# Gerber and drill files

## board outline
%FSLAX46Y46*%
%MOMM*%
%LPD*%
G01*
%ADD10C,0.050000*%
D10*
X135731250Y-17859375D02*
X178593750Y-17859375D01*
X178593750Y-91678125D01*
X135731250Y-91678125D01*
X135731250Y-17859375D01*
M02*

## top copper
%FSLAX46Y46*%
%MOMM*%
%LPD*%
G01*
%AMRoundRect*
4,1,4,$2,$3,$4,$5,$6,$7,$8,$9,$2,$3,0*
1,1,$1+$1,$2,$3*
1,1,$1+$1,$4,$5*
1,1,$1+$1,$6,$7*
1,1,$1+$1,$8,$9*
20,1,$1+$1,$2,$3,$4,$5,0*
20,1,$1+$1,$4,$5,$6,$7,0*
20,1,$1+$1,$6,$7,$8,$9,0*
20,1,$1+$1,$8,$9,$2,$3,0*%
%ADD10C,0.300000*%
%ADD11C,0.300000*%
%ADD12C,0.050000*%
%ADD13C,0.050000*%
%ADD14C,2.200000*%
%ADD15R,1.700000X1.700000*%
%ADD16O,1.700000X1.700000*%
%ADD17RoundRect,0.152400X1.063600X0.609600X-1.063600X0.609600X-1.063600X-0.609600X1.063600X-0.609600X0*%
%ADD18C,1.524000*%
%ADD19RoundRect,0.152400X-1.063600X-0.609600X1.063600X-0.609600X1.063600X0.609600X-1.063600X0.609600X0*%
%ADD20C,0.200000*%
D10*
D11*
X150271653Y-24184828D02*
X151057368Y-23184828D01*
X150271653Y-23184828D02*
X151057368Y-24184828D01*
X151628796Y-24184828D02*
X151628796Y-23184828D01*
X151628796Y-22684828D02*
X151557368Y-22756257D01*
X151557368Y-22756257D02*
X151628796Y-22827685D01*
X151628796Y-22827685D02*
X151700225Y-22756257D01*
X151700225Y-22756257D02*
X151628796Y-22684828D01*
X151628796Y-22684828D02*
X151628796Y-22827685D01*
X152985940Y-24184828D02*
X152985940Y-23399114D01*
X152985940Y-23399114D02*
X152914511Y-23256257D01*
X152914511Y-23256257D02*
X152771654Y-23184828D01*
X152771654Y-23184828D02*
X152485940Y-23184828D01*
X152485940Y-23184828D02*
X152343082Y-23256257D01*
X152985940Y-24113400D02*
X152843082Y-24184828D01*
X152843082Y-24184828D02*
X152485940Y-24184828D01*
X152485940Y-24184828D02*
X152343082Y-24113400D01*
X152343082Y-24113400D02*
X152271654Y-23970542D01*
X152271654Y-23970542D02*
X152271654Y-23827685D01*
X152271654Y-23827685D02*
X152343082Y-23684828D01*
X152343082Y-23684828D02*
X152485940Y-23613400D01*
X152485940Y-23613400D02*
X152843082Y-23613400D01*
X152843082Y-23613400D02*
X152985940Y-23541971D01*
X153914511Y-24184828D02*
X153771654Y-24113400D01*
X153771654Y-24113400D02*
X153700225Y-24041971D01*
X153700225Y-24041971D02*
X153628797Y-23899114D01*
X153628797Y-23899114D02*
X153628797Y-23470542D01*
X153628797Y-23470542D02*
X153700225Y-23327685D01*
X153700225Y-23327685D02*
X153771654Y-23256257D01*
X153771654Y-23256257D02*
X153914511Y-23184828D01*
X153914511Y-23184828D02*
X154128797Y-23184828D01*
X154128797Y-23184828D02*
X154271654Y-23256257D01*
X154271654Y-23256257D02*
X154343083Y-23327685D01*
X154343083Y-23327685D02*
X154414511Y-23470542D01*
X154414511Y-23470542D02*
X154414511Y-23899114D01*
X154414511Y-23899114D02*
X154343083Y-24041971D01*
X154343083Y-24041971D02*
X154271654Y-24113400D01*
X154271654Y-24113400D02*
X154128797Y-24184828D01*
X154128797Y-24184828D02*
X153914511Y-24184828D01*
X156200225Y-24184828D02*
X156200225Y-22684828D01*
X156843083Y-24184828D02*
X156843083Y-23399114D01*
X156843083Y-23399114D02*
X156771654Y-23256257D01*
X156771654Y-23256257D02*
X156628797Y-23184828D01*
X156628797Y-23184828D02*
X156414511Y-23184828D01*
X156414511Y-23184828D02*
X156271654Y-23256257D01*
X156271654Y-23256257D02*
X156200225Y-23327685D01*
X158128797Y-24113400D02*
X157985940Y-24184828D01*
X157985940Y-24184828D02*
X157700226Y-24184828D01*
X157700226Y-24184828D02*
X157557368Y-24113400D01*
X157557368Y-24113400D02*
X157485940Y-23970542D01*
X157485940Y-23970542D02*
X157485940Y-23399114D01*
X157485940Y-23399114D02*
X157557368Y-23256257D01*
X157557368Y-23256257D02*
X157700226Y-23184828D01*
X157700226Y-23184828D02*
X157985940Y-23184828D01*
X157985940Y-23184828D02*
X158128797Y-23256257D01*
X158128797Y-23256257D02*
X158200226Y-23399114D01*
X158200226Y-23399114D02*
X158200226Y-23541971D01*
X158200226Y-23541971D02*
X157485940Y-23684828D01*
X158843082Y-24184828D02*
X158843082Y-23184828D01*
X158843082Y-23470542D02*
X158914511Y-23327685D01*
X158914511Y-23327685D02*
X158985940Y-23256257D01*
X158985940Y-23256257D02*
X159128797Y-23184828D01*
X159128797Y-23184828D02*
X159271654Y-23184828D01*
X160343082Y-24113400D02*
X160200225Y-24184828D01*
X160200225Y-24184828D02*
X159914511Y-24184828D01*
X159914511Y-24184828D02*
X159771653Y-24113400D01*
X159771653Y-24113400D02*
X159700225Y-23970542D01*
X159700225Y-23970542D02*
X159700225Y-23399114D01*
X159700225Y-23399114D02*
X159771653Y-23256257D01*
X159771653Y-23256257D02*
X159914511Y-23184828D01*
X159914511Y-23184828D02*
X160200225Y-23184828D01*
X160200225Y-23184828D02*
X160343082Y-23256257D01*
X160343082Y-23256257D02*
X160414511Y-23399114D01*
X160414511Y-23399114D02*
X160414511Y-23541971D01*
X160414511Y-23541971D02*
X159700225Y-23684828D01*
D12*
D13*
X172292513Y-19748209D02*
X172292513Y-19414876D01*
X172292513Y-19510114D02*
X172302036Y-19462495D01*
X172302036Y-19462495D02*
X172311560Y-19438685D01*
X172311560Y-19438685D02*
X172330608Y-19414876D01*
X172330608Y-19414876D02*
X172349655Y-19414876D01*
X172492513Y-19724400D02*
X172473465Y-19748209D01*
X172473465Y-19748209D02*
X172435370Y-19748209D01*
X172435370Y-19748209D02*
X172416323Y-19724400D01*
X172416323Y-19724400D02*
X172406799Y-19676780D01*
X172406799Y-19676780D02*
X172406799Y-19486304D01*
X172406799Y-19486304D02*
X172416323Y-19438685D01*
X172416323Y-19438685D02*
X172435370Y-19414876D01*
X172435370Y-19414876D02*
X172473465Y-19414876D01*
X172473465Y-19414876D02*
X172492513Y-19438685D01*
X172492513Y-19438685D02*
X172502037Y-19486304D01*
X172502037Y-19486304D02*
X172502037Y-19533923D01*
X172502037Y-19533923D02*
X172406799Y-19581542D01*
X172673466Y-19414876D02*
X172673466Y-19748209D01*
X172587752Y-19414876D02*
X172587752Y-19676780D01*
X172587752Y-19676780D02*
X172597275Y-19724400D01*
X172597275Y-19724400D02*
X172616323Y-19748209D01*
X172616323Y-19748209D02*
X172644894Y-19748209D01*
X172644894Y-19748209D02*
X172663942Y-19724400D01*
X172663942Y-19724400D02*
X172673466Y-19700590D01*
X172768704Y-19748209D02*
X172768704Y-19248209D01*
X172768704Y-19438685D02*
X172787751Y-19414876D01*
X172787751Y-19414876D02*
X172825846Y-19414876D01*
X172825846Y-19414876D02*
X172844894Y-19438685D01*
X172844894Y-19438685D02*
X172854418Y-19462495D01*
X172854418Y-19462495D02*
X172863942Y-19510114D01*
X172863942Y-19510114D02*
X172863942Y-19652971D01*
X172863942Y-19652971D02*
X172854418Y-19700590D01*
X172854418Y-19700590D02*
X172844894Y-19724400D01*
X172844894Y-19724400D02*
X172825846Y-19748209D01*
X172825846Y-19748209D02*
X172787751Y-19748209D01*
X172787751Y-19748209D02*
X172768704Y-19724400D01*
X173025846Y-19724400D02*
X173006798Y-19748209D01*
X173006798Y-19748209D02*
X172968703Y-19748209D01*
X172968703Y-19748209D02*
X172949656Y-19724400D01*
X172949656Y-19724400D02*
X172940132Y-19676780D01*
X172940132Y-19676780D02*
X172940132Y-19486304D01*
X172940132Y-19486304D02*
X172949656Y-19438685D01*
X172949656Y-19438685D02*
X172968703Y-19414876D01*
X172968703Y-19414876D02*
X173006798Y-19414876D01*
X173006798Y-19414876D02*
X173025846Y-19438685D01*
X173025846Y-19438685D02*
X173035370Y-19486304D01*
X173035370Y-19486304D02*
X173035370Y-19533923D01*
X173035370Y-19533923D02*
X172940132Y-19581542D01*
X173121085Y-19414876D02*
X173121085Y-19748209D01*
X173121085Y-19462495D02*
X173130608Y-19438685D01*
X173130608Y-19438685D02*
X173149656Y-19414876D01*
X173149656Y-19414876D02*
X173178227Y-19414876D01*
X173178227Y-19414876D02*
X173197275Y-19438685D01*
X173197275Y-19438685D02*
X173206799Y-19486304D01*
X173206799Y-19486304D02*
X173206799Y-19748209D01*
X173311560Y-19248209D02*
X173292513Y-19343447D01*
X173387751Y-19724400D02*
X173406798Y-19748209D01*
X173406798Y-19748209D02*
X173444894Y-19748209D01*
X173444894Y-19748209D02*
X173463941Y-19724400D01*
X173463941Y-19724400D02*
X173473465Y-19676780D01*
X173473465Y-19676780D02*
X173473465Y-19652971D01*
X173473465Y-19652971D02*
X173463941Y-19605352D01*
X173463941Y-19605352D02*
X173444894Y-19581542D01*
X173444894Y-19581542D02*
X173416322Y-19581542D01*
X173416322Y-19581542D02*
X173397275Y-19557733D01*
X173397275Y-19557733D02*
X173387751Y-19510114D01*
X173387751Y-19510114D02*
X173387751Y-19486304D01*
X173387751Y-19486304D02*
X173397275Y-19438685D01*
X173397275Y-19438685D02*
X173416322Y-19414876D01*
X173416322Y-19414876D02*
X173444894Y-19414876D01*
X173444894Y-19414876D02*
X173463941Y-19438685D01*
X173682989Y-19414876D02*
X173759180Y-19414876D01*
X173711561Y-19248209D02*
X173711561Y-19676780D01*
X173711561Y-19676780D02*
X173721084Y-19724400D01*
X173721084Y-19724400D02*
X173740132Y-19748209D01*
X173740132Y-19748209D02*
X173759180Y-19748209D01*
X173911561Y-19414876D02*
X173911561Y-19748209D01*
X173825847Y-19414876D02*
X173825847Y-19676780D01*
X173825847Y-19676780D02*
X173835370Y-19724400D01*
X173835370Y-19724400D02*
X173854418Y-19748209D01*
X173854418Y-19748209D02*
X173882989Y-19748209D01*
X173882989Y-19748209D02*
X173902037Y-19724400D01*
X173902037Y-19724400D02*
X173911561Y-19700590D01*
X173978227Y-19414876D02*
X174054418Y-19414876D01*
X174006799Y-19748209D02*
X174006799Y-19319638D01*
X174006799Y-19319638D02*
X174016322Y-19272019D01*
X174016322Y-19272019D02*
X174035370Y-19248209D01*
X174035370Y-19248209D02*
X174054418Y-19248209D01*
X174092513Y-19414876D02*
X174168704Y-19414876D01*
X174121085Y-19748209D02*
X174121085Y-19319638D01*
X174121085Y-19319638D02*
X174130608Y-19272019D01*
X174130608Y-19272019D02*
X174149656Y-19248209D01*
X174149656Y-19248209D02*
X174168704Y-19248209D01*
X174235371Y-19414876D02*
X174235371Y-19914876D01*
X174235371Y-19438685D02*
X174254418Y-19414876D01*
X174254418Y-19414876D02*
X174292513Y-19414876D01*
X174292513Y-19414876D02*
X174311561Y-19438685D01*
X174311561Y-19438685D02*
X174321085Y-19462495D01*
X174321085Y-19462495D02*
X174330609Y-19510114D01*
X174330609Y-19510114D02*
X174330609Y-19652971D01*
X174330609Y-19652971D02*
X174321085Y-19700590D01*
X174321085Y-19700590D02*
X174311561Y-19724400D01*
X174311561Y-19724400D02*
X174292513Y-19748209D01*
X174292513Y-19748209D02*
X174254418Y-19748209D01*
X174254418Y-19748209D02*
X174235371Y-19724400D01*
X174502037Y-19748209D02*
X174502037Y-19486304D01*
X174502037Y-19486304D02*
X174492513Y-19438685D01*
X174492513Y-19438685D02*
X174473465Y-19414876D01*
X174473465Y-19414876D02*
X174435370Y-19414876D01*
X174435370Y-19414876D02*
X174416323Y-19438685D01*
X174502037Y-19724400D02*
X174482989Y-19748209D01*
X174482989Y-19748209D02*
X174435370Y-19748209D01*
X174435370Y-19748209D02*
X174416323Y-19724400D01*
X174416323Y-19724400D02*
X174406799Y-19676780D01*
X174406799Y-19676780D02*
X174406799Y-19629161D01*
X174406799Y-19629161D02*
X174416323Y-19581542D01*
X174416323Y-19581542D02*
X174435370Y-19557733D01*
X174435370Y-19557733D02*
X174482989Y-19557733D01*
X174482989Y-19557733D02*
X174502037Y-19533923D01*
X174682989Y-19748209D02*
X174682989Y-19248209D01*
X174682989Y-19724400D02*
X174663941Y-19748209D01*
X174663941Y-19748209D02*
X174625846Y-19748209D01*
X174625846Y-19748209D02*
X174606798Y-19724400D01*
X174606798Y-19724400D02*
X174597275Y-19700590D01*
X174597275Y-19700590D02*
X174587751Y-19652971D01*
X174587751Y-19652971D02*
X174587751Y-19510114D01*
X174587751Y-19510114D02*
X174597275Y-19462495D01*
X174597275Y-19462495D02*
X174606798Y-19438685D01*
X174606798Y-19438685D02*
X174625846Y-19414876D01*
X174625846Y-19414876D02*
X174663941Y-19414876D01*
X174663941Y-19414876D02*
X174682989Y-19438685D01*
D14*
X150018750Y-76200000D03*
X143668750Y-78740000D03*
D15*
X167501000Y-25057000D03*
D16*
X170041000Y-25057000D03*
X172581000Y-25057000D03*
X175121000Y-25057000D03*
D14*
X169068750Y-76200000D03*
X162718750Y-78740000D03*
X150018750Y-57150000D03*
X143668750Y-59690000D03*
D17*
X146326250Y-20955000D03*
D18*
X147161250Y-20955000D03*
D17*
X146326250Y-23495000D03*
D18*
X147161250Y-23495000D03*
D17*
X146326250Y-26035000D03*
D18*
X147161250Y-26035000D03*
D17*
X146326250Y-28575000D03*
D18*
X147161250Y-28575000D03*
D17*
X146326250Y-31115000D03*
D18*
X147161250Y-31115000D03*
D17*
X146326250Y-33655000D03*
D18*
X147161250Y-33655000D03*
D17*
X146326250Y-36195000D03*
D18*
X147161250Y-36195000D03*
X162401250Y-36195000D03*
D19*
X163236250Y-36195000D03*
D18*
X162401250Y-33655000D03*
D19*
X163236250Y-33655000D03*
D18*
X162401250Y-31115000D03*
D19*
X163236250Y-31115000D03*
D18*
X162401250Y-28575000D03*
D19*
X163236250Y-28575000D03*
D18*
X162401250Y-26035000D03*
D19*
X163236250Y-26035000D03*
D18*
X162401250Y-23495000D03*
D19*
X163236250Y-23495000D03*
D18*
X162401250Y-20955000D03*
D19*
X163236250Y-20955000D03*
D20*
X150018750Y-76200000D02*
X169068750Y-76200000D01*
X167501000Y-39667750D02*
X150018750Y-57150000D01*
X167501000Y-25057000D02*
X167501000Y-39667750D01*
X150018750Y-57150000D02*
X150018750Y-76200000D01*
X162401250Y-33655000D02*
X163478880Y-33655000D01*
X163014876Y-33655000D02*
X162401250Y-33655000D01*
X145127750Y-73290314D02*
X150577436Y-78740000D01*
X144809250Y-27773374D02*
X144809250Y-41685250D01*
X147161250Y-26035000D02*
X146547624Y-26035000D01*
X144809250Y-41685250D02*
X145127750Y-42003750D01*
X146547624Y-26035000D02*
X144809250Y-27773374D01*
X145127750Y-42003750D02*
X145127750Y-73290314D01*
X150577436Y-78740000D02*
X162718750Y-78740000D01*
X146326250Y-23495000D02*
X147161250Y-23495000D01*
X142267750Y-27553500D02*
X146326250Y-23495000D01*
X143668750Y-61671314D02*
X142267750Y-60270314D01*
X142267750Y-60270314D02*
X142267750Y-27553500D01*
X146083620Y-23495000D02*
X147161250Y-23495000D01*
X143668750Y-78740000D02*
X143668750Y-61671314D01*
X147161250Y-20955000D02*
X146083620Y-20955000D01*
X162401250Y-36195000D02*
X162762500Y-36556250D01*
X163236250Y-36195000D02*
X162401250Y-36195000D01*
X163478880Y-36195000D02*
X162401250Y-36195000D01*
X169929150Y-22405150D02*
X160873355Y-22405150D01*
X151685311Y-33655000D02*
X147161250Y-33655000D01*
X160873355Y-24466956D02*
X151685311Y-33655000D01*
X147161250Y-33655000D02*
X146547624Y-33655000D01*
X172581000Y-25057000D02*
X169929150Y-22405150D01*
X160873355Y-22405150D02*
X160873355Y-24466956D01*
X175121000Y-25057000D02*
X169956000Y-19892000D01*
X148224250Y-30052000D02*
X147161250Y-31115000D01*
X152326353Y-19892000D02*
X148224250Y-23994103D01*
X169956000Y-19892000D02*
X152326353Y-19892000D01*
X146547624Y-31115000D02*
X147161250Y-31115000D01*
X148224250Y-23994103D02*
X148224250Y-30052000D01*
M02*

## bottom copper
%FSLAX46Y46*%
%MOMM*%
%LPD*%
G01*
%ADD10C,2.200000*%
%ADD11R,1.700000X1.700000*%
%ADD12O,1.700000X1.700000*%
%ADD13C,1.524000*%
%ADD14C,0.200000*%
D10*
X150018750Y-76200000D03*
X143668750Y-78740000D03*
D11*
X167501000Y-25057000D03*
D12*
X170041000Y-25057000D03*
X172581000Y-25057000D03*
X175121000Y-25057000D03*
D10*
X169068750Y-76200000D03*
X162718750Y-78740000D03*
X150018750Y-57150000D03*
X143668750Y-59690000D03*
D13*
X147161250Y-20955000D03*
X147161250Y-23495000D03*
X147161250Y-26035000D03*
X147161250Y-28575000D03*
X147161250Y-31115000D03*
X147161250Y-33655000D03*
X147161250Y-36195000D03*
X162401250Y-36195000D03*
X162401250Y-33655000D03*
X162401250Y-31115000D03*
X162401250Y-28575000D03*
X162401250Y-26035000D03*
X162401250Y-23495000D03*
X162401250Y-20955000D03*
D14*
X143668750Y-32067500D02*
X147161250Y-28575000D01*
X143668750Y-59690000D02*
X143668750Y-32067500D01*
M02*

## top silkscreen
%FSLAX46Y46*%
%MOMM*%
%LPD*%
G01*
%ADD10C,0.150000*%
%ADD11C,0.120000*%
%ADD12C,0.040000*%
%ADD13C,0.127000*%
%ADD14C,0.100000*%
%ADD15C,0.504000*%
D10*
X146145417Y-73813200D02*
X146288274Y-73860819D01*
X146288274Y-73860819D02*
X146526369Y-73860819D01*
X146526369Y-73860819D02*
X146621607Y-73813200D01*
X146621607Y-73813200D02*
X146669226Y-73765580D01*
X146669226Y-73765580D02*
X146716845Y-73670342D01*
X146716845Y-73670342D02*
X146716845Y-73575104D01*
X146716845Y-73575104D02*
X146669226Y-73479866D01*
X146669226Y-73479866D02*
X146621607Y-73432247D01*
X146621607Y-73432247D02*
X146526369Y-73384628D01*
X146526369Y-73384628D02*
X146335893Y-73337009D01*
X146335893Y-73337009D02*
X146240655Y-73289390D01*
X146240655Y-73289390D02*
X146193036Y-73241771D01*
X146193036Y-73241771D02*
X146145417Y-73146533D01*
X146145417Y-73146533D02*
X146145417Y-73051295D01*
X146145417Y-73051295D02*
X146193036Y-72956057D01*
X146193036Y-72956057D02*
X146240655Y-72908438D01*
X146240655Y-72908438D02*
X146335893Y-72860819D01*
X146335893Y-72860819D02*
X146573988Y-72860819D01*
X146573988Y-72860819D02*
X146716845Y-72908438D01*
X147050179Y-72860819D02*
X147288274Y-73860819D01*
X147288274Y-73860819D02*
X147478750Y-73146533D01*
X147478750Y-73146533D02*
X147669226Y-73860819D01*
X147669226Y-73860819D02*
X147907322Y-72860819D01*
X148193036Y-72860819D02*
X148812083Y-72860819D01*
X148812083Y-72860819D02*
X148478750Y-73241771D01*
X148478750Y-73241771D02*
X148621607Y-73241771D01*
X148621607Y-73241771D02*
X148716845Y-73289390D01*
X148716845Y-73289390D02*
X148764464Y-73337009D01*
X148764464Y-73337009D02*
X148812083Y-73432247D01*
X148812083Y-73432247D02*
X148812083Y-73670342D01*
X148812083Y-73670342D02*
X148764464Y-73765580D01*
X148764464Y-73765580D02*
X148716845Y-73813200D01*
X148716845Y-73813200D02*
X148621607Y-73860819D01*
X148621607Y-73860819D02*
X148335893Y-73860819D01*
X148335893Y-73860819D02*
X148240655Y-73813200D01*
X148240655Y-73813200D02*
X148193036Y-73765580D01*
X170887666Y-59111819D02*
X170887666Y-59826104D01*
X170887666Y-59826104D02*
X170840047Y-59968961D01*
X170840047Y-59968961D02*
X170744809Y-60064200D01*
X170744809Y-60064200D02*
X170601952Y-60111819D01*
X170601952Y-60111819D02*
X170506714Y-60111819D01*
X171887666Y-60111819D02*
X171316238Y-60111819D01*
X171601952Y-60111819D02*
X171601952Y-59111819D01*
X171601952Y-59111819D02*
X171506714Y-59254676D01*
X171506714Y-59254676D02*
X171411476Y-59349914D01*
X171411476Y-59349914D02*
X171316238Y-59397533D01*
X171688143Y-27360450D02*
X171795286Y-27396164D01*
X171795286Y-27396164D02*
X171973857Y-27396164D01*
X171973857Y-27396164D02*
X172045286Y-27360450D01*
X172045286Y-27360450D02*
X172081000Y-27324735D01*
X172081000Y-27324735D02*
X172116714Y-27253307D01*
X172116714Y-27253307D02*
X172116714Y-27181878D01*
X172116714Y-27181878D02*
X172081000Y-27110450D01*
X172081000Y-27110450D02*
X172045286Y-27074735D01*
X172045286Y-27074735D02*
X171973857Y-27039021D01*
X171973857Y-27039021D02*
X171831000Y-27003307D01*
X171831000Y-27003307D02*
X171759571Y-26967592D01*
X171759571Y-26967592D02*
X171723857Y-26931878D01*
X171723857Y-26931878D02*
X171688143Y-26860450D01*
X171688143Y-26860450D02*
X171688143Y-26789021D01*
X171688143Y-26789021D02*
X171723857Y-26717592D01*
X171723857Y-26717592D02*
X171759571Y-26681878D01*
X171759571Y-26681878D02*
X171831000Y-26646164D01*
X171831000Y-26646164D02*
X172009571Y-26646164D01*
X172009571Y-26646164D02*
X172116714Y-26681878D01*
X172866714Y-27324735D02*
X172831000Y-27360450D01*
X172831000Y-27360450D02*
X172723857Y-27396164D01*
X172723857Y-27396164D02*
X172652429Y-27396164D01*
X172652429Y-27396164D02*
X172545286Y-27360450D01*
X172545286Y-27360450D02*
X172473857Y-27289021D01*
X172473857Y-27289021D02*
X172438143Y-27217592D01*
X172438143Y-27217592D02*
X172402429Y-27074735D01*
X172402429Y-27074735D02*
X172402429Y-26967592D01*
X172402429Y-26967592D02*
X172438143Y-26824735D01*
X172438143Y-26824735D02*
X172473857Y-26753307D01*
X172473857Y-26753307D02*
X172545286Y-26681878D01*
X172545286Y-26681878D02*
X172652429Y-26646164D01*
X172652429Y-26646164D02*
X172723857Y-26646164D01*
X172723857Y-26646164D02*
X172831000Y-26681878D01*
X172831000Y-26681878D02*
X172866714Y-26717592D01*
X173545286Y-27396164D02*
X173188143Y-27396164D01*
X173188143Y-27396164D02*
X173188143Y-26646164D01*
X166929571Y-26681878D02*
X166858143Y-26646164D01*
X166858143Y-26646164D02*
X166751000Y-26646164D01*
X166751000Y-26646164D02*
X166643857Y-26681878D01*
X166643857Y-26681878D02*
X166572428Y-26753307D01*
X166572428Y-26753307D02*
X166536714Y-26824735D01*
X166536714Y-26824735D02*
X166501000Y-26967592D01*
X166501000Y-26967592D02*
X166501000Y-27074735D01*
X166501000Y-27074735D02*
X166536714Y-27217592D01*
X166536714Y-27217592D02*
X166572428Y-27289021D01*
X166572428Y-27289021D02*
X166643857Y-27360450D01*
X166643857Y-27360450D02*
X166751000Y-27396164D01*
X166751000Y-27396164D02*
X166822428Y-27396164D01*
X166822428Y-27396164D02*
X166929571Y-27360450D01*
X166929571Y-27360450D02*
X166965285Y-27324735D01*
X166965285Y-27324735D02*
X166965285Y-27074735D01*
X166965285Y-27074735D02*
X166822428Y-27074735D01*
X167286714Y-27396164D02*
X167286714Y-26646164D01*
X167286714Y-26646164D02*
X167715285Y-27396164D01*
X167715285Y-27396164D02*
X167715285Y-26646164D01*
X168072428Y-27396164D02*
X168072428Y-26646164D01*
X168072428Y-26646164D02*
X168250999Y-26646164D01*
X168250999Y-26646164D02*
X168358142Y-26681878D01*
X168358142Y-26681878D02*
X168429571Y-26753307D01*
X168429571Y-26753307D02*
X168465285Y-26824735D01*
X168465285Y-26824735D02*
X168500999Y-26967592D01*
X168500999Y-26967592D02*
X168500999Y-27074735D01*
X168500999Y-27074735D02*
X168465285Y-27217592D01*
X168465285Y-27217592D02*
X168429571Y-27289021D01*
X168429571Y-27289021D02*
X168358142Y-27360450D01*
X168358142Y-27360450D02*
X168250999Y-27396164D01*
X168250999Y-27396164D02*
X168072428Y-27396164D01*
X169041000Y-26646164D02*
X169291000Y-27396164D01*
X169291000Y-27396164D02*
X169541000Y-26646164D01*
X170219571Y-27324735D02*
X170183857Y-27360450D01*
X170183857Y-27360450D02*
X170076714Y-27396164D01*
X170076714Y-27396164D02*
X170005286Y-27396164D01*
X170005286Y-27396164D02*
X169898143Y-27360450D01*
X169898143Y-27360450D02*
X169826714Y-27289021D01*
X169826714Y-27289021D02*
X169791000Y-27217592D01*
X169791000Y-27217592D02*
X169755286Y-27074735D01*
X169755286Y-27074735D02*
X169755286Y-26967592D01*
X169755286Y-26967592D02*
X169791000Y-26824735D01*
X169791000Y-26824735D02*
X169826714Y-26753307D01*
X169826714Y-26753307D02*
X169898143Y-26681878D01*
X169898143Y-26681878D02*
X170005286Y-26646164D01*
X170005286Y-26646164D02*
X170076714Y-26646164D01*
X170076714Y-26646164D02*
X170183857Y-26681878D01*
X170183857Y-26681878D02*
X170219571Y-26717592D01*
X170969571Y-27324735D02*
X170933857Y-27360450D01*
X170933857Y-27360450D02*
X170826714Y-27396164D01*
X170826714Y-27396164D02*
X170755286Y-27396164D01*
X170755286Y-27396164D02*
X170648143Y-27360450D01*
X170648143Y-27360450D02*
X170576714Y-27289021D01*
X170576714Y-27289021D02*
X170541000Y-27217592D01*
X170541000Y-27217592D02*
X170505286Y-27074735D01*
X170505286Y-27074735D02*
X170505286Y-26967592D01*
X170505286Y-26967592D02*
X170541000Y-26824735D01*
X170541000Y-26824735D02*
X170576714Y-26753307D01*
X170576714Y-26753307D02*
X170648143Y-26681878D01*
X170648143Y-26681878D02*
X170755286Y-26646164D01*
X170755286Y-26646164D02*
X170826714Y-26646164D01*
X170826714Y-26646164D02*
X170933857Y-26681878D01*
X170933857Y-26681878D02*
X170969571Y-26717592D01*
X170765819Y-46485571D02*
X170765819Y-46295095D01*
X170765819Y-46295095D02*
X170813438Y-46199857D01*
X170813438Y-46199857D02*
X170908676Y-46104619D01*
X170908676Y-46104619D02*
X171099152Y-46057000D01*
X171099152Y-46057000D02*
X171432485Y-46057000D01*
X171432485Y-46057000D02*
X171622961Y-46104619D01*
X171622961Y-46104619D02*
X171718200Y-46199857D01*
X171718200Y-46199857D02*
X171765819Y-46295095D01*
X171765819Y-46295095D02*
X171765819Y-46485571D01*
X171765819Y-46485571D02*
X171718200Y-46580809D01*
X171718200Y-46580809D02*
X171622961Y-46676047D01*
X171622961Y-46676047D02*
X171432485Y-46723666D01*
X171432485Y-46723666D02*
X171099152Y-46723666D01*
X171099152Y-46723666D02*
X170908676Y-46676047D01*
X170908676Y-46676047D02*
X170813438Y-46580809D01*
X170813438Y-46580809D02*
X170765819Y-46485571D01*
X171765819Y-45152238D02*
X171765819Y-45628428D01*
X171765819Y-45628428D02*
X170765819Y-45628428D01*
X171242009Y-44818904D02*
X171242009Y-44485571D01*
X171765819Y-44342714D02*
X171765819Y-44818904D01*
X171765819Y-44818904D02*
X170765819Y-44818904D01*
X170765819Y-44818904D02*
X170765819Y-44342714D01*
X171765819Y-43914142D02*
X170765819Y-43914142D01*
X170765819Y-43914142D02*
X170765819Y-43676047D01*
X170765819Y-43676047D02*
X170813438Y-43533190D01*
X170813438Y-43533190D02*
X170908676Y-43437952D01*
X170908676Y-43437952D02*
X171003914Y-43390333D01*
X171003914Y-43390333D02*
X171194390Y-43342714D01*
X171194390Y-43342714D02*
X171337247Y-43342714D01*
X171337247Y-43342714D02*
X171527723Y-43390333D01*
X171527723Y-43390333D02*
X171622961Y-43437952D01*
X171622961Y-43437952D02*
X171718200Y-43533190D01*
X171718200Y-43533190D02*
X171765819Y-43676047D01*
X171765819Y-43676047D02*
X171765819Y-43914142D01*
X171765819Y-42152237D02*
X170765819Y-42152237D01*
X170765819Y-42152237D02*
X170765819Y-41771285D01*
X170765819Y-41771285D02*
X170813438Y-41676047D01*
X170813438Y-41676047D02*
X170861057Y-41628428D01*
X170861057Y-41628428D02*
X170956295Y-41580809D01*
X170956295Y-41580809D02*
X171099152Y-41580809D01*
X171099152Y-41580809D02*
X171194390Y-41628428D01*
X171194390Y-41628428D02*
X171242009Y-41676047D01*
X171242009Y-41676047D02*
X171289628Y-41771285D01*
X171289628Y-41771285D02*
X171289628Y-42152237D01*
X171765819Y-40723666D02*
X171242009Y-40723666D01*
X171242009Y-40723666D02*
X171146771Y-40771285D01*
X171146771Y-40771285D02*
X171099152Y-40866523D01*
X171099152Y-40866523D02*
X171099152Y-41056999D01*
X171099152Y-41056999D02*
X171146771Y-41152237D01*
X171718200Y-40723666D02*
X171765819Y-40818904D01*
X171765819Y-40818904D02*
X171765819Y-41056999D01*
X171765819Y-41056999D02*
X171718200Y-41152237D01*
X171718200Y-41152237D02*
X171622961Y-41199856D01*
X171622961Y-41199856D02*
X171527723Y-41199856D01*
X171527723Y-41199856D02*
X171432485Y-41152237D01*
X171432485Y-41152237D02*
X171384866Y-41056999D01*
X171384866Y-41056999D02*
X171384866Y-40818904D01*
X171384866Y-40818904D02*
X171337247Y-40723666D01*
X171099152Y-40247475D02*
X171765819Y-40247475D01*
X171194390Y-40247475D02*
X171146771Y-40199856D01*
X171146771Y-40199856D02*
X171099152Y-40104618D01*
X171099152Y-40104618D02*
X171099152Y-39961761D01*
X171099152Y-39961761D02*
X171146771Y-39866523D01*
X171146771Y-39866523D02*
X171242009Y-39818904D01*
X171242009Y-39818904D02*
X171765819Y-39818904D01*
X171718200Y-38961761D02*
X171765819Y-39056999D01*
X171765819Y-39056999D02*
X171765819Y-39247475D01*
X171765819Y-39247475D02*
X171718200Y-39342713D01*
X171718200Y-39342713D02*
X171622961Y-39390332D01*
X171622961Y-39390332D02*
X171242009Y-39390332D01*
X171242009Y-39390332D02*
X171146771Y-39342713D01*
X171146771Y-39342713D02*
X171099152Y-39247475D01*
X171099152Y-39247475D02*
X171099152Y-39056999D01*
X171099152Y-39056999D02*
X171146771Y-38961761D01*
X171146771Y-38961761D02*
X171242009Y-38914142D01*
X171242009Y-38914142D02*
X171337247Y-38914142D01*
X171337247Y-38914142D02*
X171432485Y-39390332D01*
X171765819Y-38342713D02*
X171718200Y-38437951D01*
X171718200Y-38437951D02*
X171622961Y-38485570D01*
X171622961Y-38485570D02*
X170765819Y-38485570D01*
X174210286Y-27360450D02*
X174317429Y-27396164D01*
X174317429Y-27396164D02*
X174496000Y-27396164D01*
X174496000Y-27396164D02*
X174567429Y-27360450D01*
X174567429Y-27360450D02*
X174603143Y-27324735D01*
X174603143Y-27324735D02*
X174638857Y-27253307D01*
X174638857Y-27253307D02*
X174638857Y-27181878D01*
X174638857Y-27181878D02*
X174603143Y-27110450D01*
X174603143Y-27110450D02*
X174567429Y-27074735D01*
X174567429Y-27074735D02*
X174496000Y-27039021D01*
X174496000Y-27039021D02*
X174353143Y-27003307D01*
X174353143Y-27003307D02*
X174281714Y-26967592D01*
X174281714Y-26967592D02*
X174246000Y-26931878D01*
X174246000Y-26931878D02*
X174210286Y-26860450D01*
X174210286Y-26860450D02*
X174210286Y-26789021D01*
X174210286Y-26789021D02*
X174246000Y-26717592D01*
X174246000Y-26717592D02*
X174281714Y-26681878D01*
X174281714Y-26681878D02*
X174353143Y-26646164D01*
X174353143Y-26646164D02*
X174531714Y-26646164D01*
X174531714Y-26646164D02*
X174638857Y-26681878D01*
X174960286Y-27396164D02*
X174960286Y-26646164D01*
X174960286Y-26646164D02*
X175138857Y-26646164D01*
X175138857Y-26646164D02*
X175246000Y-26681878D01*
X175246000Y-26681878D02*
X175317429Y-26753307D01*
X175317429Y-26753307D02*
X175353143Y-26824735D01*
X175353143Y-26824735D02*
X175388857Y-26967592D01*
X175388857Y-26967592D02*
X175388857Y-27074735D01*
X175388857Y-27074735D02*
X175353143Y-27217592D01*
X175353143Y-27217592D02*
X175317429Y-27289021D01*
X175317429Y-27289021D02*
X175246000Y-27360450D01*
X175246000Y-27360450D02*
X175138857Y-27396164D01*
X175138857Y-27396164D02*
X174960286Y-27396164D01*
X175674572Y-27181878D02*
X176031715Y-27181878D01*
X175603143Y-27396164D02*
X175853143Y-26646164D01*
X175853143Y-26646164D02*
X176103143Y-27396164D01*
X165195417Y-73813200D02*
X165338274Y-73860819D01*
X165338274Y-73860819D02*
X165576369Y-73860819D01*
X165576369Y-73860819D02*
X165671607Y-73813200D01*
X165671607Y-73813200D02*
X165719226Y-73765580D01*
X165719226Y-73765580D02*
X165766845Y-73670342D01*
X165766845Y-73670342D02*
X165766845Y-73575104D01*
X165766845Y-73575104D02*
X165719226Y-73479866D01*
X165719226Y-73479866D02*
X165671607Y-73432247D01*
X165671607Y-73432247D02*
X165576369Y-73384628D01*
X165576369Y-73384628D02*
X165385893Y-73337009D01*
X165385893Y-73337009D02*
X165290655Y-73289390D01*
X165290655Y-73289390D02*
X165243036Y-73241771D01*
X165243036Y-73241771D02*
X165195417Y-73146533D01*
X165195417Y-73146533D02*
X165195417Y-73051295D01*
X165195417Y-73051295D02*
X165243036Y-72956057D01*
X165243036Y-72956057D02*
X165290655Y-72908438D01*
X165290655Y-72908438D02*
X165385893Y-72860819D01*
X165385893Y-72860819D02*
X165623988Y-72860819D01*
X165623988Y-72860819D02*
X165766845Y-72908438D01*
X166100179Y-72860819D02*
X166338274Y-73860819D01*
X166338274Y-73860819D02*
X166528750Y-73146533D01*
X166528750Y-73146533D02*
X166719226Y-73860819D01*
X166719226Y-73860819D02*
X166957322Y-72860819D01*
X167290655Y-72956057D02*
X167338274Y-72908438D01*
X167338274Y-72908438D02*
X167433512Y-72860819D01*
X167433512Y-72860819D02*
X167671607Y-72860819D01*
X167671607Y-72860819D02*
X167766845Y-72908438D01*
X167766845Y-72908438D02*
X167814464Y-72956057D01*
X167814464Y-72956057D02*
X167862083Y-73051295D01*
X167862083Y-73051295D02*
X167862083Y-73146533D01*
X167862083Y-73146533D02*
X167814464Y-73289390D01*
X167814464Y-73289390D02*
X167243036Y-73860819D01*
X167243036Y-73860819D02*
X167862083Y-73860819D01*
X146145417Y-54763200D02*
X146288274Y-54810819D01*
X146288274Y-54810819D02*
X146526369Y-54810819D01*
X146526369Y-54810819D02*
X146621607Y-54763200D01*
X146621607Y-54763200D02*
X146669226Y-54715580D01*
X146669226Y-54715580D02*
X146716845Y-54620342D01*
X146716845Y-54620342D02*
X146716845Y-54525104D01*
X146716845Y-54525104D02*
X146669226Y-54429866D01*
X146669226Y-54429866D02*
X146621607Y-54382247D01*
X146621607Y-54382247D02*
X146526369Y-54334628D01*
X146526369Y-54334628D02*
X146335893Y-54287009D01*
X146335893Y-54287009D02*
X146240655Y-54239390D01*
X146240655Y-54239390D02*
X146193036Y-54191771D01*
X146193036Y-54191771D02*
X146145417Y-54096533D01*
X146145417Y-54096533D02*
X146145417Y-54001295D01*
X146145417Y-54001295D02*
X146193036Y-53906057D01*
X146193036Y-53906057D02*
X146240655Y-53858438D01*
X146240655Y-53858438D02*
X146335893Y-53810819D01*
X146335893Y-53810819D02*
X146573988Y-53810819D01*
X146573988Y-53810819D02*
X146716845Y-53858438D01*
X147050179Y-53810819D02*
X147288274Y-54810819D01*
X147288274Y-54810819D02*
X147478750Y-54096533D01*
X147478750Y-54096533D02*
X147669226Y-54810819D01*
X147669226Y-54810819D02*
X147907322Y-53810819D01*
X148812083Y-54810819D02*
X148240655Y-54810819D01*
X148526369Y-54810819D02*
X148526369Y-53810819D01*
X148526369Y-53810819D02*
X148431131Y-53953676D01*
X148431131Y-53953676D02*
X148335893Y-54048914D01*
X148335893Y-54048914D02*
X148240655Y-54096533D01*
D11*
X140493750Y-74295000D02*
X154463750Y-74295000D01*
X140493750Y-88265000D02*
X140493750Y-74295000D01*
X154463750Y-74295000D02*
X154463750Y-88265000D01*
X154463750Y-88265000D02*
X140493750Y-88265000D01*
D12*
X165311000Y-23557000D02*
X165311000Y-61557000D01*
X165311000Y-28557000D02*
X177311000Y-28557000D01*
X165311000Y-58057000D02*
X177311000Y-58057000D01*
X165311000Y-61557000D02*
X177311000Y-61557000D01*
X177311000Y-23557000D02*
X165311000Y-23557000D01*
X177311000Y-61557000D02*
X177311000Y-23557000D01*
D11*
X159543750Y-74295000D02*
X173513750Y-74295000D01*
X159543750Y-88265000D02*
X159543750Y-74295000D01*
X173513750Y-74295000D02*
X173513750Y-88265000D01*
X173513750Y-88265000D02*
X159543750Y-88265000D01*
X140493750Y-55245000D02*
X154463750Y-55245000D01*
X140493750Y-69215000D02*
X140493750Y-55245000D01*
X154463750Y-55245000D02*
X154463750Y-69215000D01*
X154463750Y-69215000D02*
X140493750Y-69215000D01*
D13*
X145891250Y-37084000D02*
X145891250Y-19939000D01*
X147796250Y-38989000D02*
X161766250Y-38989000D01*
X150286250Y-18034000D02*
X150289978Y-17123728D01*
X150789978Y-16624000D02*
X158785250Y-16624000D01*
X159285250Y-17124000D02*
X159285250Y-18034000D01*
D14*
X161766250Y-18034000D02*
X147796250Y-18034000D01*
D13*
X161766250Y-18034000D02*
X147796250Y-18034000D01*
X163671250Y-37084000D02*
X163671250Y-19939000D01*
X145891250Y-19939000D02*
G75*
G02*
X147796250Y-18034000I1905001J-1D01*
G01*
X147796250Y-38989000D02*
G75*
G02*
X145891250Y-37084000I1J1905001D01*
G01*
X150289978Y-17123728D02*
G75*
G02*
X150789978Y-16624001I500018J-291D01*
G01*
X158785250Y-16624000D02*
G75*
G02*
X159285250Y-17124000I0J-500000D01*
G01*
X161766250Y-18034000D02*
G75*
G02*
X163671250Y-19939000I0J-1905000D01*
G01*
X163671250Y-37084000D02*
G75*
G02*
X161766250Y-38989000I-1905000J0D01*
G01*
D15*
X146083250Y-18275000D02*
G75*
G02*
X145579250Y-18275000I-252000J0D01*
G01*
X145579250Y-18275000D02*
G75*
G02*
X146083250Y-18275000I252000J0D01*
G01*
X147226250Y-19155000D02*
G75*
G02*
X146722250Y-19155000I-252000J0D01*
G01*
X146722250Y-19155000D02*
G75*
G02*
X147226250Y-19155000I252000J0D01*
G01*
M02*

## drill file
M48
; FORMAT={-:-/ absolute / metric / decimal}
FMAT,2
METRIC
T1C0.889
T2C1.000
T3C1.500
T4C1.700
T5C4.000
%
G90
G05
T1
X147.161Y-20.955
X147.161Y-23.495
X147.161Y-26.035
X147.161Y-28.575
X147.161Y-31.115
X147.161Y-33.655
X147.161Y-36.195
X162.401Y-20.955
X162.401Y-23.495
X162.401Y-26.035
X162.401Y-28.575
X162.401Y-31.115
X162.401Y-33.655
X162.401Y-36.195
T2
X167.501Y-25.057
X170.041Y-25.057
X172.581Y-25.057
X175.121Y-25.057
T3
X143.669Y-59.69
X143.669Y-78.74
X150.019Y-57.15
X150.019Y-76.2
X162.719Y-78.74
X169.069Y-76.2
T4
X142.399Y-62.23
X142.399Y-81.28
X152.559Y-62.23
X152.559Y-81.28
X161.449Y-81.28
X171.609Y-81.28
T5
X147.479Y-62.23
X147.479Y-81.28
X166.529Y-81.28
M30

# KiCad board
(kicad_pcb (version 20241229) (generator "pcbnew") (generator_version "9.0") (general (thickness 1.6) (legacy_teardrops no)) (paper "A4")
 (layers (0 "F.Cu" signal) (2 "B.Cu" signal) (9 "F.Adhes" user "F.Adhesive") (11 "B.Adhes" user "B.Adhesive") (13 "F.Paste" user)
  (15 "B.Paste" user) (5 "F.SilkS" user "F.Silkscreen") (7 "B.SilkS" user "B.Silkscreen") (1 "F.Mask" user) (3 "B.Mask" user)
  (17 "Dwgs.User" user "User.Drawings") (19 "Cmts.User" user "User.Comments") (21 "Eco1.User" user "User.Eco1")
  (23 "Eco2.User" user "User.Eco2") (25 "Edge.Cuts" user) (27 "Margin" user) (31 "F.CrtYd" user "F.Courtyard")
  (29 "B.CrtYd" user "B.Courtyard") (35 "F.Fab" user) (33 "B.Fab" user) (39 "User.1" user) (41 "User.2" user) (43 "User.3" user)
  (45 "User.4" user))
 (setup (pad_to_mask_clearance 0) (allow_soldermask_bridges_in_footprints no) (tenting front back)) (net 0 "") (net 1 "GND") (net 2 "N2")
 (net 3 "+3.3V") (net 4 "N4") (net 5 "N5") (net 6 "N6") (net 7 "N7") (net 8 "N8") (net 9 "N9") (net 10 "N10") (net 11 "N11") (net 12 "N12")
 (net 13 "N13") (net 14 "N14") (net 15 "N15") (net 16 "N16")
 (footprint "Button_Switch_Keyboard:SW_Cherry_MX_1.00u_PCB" (layer "F.Cu") (at 150.01875 76.2)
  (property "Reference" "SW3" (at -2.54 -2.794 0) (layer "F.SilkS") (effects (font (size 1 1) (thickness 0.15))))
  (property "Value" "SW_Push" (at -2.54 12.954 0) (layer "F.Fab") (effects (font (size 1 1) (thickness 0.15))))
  (fp_line (start -9.525 -1.905) (end 4.445 -1.905) (stroke (width 0.12) (type solid)) (layer "F.SilkS"))
  (fp_line (start -9.525 12.065) (end -9.525 -1.905) (stroke (width 0.12) (type solid)) (layer "F.SilkS"))
  (fp_line (start 4.445 -1.905) (end 4.445 12.065) (stroke (width 0.12) (type solid)) (layer "F.SilkS"))
  (fp_line (start 4.445 12.065) (end -9.525 12.065) (stroke (width 0.12) (type solid)) (layer "F.SilkS"))
  (pad "" np_thru_hole circle (at -7.62 5.08) (size 1.7 1.7) (drill 1.7) (layers "*.Cu" "*.Mask"))
  (pad "" np_thru_hole circle (at -2.54 5.08) (size 4 4) (drill 4) (layers "*.Cu" "*.Mask"))
  (pad "" np_thru_hole circle (at 2.54 5.08) (size 1.7 1.7) (drill 1.7) (layers "*.Cu" "*.Mask"))
  (pad "1" thru_hole circle (at 0 0) (size 2.2 2.2) (drill 1.5) (layers "*.Cu" "*.Mask") (remove_unused_layers no) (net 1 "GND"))
  (pad "2" thru_hole circle (at -6.35 2.54) (size 2.2 2.2) (drill 1.5) (layers "*.Cu" "*.Mask") (remove_unused_layers no) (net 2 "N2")))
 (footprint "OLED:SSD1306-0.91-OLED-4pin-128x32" (layer "F.Cu") (at 165.311 61.557 90)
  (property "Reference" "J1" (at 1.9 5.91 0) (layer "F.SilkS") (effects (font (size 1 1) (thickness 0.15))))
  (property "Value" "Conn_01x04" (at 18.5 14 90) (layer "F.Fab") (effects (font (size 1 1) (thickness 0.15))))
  (fp_line (start 38 0) (end 0 0) (stroke (width 0.04) (type solid)) (layer "F.SilkS"))
  (fp_line (start 33 0) (end 33 12) (stroke (width 0.04) (type solid)) (layer "F.SilkS"))
  (fp_line (start 3.5 0) (end 3.5 12) (stroke (width 0.04) (type solid)) (layer "F.SilkS"))
  (fp_line (start 0 0) (end 0 12) (stroke (width 0.04) (type solid)) (layer "F.SilkS"))
  (fp_line (start 38 12) (end 38 0) (stroke (width 0.04) (type solid)) (layer "F.SilkS"))
  (fp_line (start 0 12) (end 38 12) (stroke (width 0.04) (type solid)) (layer "F.SilkS"))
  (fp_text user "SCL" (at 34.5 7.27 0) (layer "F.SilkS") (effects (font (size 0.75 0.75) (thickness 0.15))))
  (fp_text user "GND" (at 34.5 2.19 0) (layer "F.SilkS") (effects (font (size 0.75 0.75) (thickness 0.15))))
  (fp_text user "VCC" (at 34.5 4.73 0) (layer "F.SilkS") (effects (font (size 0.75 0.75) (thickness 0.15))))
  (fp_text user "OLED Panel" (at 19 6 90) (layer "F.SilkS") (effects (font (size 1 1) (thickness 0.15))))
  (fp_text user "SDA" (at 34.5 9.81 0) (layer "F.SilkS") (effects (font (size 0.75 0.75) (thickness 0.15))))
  (pad "1" thru_hole rect (at 36.5 2.19 90) (size 1.7 1.7) (drill 1) (layers "*.Cu" "*.Mask") (remove_unused_layers no) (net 1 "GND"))
  (pad "2" thru_hole oval (at 36.5 4.73 90) (size 1.7 1.7) (drill 1) (layers "*.Cu" "*.Mask") (remove_unused_layers no) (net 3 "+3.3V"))
  (pad "3" thru_hole oval (at 36.5 7.27 90) (size 1.7 1.7) (drill 1) (layers "*.Cu" "*.Mask") (remove_unused_layers no) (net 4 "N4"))
  (pad "4" thru_hole oval (at 36.5 9.81 90) (size 1.7 1.7) (drill 1) (layers "*.Cu" "*.Mask") (remove_unused_layers no) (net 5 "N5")))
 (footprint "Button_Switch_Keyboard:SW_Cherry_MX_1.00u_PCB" (layer "F.Cu") (at 169.06875 76.2)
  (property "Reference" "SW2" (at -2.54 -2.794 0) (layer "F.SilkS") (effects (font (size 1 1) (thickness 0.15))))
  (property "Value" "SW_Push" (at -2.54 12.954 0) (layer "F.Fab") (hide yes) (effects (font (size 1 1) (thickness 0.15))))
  (fp_line (start -9.525 -1.905) (end 4.445 -1.905) (stroke (width 0.12) (type solid)) (layer "F.SilkS"))
  (fp_line (start -9.525 12.065) (end -9.525 -1.905) (stroke (width 0.12) (type solid)) (layer "F.SilkS"))
  (fp_line (start 4.445 -1.905) (end 4.445 12.065) (stroke (width 0.12) (type solid)) (layer "F.SilkS"))
  (fp_line (start 4.445 12.065) (end -9.525 12.065) (stroke (width 0.12) (type solid)) (layer "F.SilkS"))
  (pad "" np_thru_hole circle (at -7.62 5.08) (size 1.7 1.7) (drill 1.7) (layers "*.Cu" "*.Mask"))
  (pad "" np_thru_hole circle (at -2.54 5.08) (size 4 4) (drill 4) (layers "*.Cu" "*.Mask"))
  (pad "" np_thru_hole circle (at 2.54 5.08) (size 1.7 1.7) (drill 1.7) (layers "*.Cu" "*.Mask"))
  (pad "1" thru_hole circle (at 0 0) (size 2.2 2.2) (drill 1.5) (layers "*.Cu" "*.Mask") (remove_unused_layers no) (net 1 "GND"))
  (pad "2" thru_hole circle (at -6.35 2.54) (size 2.2 2.2) (drill 1.5) (layers "*.Cu" "*.Mask") (remove_unused_layers no) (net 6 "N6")))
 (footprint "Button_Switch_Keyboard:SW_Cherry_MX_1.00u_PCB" (layer "F.Cu") (at 150.01875 57.15)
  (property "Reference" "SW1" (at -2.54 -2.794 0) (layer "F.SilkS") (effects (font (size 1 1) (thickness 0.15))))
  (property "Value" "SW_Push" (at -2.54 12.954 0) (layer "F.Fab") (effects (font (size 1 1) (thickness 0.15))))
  (fp_line (start -9.525 -1.905) (end 4.445 -1.905) (stroke (width 0.12) (type solid)) (layer "F.SilkS"))
  (fp_line (start -9.525 12.065) (end -9.525 -1.905) (stroke (width 0.12) (type solid)) (layer "F.SilkS"))
  (fp_line (start 4.445 -1.905) (end 4.445 12.065) (stroke (width 0.12) (type solid)) (layer "F.SilkS"))
  (fp_line (start 4.445 12.065) (end -9.525 12.065) (stroke (width 0.12) (type solid)) (layer "F.SilkS"))
  (pad "" np_thru_hole circle (at -7.62 5.08) (size 1.7 1.7) (drill 1.7) (layers "*.Cu" "*.Mask"))
  (pad "" np_thru_hole circle (at -2.54 5.08) (size 4 4) (drill 4) (layers "*.Cu" "*.Mask"))
  (pad "" np_thru_hole circle (at 2.54 5.08) (size 1.7 1.7) (drill 1.7) (layers "*.Cu" "*.Mask"))
  (pad "1" thru_hole circle (at 0 0) (size 2.2 2.2) (drill 1.5) (layers "*.Cu" "*.Mask") (remove_unused_layers no) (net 1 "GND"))
  (pad "2" thru_hole circle (at -6.35 2.54) (size 2.2 2.2) (drill 1.5) (layers "*.Cu" "*.Mask") (remove_unused_layers no) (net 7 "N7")))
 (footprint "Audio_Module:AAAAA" (layer "F.Cu") (at 154.78125 28.575)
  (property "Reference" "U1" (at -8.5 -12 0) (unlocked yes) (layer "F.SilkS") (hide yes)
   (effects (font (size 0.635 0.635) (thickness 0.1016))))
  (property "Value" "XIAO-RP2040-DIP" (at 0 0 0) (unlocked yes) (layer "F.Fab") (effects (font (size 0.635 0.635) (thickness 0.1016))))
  (fp_line (start -8.89 8.509) (end -8.89 -8.636) (stroke (width 0.127) (type solid)) (layer "F.SilkS"))
  (fp_line (start -6.985 10.414) (end 6.985 10.414) (stroke (width 0.127) (type solid)) (layer "F.SilkS"))
  (fp_line (start -4.495 -10.541) (end -4.491272 -11.451272) (stroke (width 0.127) (type solid)) (layer "F.SilkS"))
  (fp_line (start -3.991272 -11.951) (end 4.004 -11.951) (stroke (width 0.127) (type solid)) (layer "F.SilkS"))
  (fp_line (start 4.504 -11.451) (end 4.504 -10.541) (stroke (width 0.127) (type solid)) (layer "F.SilkS"))
  (fp_line (start 6.985 -10.541) (end -6.985 -10.541) (stroke (width 0.1) (type solid)) (layer "F.SilkS"))
  (fp_line (start 6.985 -10.541) (end -6.985 -10.541) (stroke (width 0.127) (type solid)) (layer "F.SilkS"))
  (fp_line (start 8.89 8.509) (end 8.89 -8.636) (stroke (width 0.127) (type solid)) (layer "F.SilkS"))
  (fp_arc (start -8.89 -8.636) (mid -8.332038 -9.983038) (end -6.985 -10.541) (stroke (width 0.127) (type solid)) (layer "F.SilkS"))
  (fp_arc (start -6.985 10.414) (mid -8.332038 9.856038) (end -8.89 8.509) (stroke (width 0.127) (type solid)) (layer "F.SilkS"))
  (fp_arc (start -4.491272 -11.451272) (mid -4.344728 -11.80464) (end -3.991272 -11.951) (stroke (width 0.127) (type default))
   (layer "F.SilkS"))
  (fp_arc (start 4.004 -11.951) (mid 4.357553 -11.804553) (end 4.504 -11.451) (stroke (width 0.127) (type default)) (layer "F.SilkS"))
  (fp_arc (start 6.985 -10.541) (mid 8.332038 -9.983038) (end 8.89 -8.636) (stroke (width 0.127) (type solid)) (layer "F.SilkS"))
  (fp_arc (start 8.89 8.509) (mid 8.332038 9.856038) (end 6.985 10.414) (stroke (width 0.127) (type solid)) (layer "F.SilkS"))
  (fp_circle (center -8.95 -10.3) (end -8.95 -10.554) (stroke (width 0.5) (type solid)) (fill yes) (layer "F.SilkS"))
  (fp_circle (center -7.807 -9.42) (end -7.807 -9.674) (stroke (width 0.5) (type solid)) (fill yes) (layer "F.SilkS"))
  (pad "1" smd roundrect (at -8.455 -7.62 180) (size 2.432 1.524) (layers "F.Cu" "F.Mask") (roundrect_rratio 0.1) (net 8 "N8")
   (thermal_bridge_angle 45))
  (pad "1" thru_hole circle (at -7.62 -7.62 180) (size 1.524 1.524) (drill 0.889) (layers "*.Cu" "*.Mask") (remove_unused_layers no)
   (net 8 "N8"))
  (pad "2" smd roundrect (at -8.455 -5.08 180) (size 2.432 1.524) (layers "F.Cu" "F.Mask") (roundrect_rratio 0.1) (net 2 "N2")
   (thermal_bridge_angle 45))
  (pad "2" thru_hole circle (at -7.62 -5.08 180) (size 1.524 1.524) (drill 0.889) (layers "*.Cu" "*.Mask") (remove_unused_layers no)
   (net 2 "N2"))
  (pad "3" smd roundrect (at -8.455 -2.54 180) (size 2.432 1.524) (layers "F.Cu" "F.Mask") (roundrect_rratio 0.1) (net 6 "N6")
   (thermal_bridge_angle 45))
  (pad "3" thru_hole circle (at -7.62 -2.54 180) (size 1.524 1.524) (drill 0.889) (layers "*.Cu" "*.Mask") (remove_unused_layers no)
   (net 6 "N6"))
  (pad "4" smd roundrect (at -8.455 0 180) (size 2.432 1.524) (layers "F.Cu" "F.Mask") (roundrect_rratio 0.1) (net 7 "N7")
   (thermal_bridge_angle 45))
  (pad "4" thru_hole circle (at -7.62 0 180) (size 1.524 1.524) (drill 0.889) (layers "*.Cu" "*.Mask") (remove_unused_layers no)
   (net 7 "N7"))
  (pad "5" smd roundrect (at -8.455 2.54 180) (size 2.432 1.524) (layers "F.Cu" "F.Mask") (roundrect_rratio 0.1) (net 5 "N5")
   (thermal_bridge_angle 45))
  (pad "5" thru_hole circle (at -7.62 2.54 180) (size 1.524 1.524) (drill 0.889) (layers "*.Cu" "*.Mask") (remove_unused_layers no)
   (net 5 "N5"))
  (pad "6" smd roundrect (at -8.455 5.08 180) (size 2.432 1.524) (layers "F.Cu" "F.Mask") (roundrect_rratio 0.1) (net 4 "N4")
   (thermal_bridge_angle 45))
  (pad "6" thru_hole circle (at -7.62 5.08 180) (size 1.524 1.524) (drill 0.889) (layers "*.Cu" "*.Mask") (remove_unused_layers no)
   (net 4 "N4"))
  (pad "7" smd roundrect (at -8.455 7.62 180) (size 2.432 1.524) (layers "F.Cu" "F.Mask") (roundrect_rratio 0.1) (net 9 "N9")
   (thermal_bridge_angle 45))
  (pad "7" thru_hole circle (at -7.62 7.62 180) (size 1.524 1.524) (drill 0.889) (layers "*.Cu" "*.Mask") (remove_unused_layers no)
   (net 9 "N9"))
  (pad "8" thru_hole circle (at 7.62 7.62) (size 1.524 1.524) (drill 0.889) (layers "*.Cu" "*.Mask") (remove_unused_layers no)
   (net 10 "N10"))
  (pad "8" smd roundrect (at 8.455 7.62) (size 2.432 1.524) (layers "F.Cu" "F.Mask") (roundrect_rratio 0.1) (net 10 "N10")
   (thermal_bridge_angle 45))
  (pad "9" thru_hole circle (at 7.62 5.08) (size 1.524 1.524) (drill 0.889) (layers "*.Cu" "*.Mask") (remove_unused_layers no)
   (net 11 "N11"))
  (pad "9" smd roundrect (at 8.455 5.08) (size 2.432 1.524) (layers "F.Cu" "F.Mask") (roundrect_rratio 0.1) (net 11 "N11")
   (thermal_bridge_angle 45))
  (pad "10" thru_hole circle (at 7.62 2.54) (size 1.524 1.524) (drill 0.889) (layers "*.Cu" "*.Mask") (remove_unused_layers no)
   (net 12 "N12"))
  (pad "10" smd roundrect (at 8.455 2.54) (size 2.432 1.524) (layers "F.Cu" "F.Mask") (roundrect_rratio 0.1) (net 12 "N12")
   (thermal_bridge_angle 45))
  (pad "11" thru_hole circle (at 7.62 0) (size 1.524 1.524) (drill 0.889) (layers "*.Cu" "*.Mask") (remove_unused_layers no) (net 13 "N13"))
  (pad "11" smd roundrect (at 8.455 0) (size 2.432 1.524) (layers "F.Cu" "F.Mask") (roundrect_rratio 0.1) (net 13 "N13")
   (thermal_bridge_angle 45))
  (pad "12" thru_hole circle (at 7.62 -2.54) (size 1.524 1.524) (drill 0.889) (layers "*.Cu" "*.Mask") (remove_unused_layers no)
   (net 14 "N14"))
  (pad "12" smd roundrect (at 8.455 -2.54) (size 2.432 1.524) (layers "F.Cu" "F.Mask") (roundrect_rratio 0.1) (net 14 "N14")
   (thermal_bridge_angle 45))
  (pad "13" thru_hole circle (at 7.62 -5.08) (size 1.524 1.524) (drill 0.889) (layers "*.Cu" "*.Mask") (remove_unused_layers no)
   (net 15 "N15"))
  (pad "13" smd roundrect (at 8.455 -5.08) (size 2.432 1.524) (layers "F.Cu" "F.Mask") (roundrect_rratio 0.1) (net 15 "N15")
   (thermal_bridge_angle 45))
  (pad "14" thru_hole circle (at 7.62 -7.62) (size 1.524 1.524) (drill 0.889) (layers "*.Cu" "*.Mask") (remove_unused_layers no)
   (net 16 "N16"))
  (pad "14" smd roundrect (at 8.455 -7.62) (size 2.432 1.524) (layers "F.Cu" "F.Mask") (roundrect_rratio 0.1) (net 16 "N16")
   (thermal_bridge_angle 45)))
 (gr_rect (start 135.73125 17.859375) (end 178.59375 91.678125) (stroke (width 0.05) (type default)) (fill no) (layer "Edge.Cuts"))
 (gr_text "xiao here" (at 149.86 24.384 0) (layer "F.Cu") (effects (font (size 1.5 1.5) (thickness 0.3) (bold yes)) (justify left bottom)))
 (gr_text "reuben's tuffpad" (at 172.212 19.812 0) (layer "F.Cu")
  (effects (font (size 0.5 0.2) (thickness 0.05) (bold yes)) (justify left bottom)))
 (segment (start 150.01875 76.2) (end 169.06875 76.2) (width 0.2) (layer "F.Cu") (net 1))
 (segment (start 167.501 39.66775) (end 150.01875 57.15) (width 0.2) (layer "F.Cu") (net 1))
 (segment (start 167.501 25.057) (end 167.501 39.66775) (width 0.2) (layer "F.Cu") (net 1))
 (segment (start 150.01875 57.15) (end 150.01875 76.2) (width 0.2) (layer "F.Cu") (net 1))
 (segment (start 162.40125 33.655) (end 163.47888 33.655) (width 0.2) (layer "F.Cu") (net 11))
 (segment (start 163.014876 33.655) (end 162.40125 33.655) (width 0.2) (layer "F.Cu") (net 11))
 (segment (start 143.66875 32.0675) (end 147.16125 28.575) (width 0.2) (layer "B.Cu") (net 7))
 (segment (start 143.66875 59.69) (end 143.66875 32.0675) (width 0.2) (layer "B.Cu") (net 7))
 (segment (start 145.12775 73.290314) (end 150.577436 78.74) (width 0.2) (layer "F.Cu") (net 6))
 (segment (start 144.80925 27.773374) (end 144.80925 41.68525) (width 0.2) (layer "F.Cu") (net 6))
 (segment (start 147.16125 26.035) (end 146.547624 26.035) (width 0.2) (layer "F.Cu") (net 6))
 (segment (start 144.80925 41.68525) (end 145.12775 42.00375) (width 0.2) (layer "F.Cu") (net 6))
 (segment (start 146.547624 26.035) (end 144.80925 27.773374) (width 0.2) (layer "F.Cu") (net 6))
 (segment (start 145.12775 42.00375) (end 145.12775 73.290314) (width 0.2) (layer "F.Cu") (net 6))
 (segment (start 150.577436 78.74) (end 162.71875 78.74) (width 0.2) (layer "F.Cu") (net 6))
 (segment (start 146.32625 23.495) (end 147.16125 23.495) (width 0.2) (layer "F.Cu") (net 2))
 (segment (start 142.26775 27.5535) (end 146.32625 23.495) (width 0.2) (layer "F.Cu") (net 2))
 (segment (start 143.66875 61.671314) (end 142.26775 60.270314) (width 0.2) (layer "F.Cu") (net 2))
 (segment (start 142.26775 60.270314) (end 142.26775 27.5535) (width 0.2) (layer "F.Cu") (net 2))
 (segment (start 146.08362 23.495) (end 147.16125 23.495) (width 0.2) (layer "F.Cu") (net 2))
 (segment (start 143.66875 78.74) (end 143.66875 61.671314) (width 0.2) (layer "F.Cu") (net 2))
 (segment (start 147.16125 20.955) (end 146.08362 20.955) (width 0.2) (layer "F.Cu") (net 8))
 (segment (start 162.40125 36.195) (end 162.7625 36.55625) (width 0.2) (layer "F.Cu") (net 10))
 (segment (start 163.23625 36.195) (end 162.40125 36.195) (width 0.2) (layer "F.Cu") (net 10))
 (segment (start 163.47888 36.195) (end 162.40125 36.195) (width 0.2) (layer "F.Cu") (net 10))
 (segment (start 169.92915 22.40515) (end 160.873355 22.40515) (width 0.2) (layer "F.Cu") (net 4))
 (segment (start 151.685311 33.655) (end 147.16125 33.655) (width 0.2) (layer "F.Cu") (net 4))
 (segment (start 160.873355 24.466956) (end 151.685311 33.655) (width 0.2) (layer "F.Cu") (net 4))
 (segment (start 147.16125 33.655) (end 146.547624 33.655) (width 0.2) (layer "F.Cu") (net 4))
 (segment (start 172.581 25.057) (end 169.92915 22.40515) (width 0.2) (layer "F.Cu") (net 4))
 (segment (start 160.873355 22.40515) (end 160.873355 24.466956) (width 0.2) (layer "F.Cu") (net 4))
 (segment (start 175.121 25.057) (end 169.956 19.892) (width 0.2) (layer "F.Cu") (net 5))
 (segment (start 148.22425 30.052) (end 147.16125 31.115) (width 0.2) (layer "F.Cu") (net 5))
 (segment (start 152.326353 19.892) (end 148.22425 23.994103) (width 0.2) (layer "F.Cu") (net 5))
 (segment (start 169.956 19.892) (end 152.326353 19.892) (width 0.2) (layer "F.Cu") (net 5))
 (segment (start 146.547624 31.115) (end 147.16125 31.115) (width 0.2) (layer "F.Cu") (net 5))
 (segment (start 148.22425 23.994103) (end 148.22425 30.052) (width 0.2) (layer "F.Cu") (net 5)))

